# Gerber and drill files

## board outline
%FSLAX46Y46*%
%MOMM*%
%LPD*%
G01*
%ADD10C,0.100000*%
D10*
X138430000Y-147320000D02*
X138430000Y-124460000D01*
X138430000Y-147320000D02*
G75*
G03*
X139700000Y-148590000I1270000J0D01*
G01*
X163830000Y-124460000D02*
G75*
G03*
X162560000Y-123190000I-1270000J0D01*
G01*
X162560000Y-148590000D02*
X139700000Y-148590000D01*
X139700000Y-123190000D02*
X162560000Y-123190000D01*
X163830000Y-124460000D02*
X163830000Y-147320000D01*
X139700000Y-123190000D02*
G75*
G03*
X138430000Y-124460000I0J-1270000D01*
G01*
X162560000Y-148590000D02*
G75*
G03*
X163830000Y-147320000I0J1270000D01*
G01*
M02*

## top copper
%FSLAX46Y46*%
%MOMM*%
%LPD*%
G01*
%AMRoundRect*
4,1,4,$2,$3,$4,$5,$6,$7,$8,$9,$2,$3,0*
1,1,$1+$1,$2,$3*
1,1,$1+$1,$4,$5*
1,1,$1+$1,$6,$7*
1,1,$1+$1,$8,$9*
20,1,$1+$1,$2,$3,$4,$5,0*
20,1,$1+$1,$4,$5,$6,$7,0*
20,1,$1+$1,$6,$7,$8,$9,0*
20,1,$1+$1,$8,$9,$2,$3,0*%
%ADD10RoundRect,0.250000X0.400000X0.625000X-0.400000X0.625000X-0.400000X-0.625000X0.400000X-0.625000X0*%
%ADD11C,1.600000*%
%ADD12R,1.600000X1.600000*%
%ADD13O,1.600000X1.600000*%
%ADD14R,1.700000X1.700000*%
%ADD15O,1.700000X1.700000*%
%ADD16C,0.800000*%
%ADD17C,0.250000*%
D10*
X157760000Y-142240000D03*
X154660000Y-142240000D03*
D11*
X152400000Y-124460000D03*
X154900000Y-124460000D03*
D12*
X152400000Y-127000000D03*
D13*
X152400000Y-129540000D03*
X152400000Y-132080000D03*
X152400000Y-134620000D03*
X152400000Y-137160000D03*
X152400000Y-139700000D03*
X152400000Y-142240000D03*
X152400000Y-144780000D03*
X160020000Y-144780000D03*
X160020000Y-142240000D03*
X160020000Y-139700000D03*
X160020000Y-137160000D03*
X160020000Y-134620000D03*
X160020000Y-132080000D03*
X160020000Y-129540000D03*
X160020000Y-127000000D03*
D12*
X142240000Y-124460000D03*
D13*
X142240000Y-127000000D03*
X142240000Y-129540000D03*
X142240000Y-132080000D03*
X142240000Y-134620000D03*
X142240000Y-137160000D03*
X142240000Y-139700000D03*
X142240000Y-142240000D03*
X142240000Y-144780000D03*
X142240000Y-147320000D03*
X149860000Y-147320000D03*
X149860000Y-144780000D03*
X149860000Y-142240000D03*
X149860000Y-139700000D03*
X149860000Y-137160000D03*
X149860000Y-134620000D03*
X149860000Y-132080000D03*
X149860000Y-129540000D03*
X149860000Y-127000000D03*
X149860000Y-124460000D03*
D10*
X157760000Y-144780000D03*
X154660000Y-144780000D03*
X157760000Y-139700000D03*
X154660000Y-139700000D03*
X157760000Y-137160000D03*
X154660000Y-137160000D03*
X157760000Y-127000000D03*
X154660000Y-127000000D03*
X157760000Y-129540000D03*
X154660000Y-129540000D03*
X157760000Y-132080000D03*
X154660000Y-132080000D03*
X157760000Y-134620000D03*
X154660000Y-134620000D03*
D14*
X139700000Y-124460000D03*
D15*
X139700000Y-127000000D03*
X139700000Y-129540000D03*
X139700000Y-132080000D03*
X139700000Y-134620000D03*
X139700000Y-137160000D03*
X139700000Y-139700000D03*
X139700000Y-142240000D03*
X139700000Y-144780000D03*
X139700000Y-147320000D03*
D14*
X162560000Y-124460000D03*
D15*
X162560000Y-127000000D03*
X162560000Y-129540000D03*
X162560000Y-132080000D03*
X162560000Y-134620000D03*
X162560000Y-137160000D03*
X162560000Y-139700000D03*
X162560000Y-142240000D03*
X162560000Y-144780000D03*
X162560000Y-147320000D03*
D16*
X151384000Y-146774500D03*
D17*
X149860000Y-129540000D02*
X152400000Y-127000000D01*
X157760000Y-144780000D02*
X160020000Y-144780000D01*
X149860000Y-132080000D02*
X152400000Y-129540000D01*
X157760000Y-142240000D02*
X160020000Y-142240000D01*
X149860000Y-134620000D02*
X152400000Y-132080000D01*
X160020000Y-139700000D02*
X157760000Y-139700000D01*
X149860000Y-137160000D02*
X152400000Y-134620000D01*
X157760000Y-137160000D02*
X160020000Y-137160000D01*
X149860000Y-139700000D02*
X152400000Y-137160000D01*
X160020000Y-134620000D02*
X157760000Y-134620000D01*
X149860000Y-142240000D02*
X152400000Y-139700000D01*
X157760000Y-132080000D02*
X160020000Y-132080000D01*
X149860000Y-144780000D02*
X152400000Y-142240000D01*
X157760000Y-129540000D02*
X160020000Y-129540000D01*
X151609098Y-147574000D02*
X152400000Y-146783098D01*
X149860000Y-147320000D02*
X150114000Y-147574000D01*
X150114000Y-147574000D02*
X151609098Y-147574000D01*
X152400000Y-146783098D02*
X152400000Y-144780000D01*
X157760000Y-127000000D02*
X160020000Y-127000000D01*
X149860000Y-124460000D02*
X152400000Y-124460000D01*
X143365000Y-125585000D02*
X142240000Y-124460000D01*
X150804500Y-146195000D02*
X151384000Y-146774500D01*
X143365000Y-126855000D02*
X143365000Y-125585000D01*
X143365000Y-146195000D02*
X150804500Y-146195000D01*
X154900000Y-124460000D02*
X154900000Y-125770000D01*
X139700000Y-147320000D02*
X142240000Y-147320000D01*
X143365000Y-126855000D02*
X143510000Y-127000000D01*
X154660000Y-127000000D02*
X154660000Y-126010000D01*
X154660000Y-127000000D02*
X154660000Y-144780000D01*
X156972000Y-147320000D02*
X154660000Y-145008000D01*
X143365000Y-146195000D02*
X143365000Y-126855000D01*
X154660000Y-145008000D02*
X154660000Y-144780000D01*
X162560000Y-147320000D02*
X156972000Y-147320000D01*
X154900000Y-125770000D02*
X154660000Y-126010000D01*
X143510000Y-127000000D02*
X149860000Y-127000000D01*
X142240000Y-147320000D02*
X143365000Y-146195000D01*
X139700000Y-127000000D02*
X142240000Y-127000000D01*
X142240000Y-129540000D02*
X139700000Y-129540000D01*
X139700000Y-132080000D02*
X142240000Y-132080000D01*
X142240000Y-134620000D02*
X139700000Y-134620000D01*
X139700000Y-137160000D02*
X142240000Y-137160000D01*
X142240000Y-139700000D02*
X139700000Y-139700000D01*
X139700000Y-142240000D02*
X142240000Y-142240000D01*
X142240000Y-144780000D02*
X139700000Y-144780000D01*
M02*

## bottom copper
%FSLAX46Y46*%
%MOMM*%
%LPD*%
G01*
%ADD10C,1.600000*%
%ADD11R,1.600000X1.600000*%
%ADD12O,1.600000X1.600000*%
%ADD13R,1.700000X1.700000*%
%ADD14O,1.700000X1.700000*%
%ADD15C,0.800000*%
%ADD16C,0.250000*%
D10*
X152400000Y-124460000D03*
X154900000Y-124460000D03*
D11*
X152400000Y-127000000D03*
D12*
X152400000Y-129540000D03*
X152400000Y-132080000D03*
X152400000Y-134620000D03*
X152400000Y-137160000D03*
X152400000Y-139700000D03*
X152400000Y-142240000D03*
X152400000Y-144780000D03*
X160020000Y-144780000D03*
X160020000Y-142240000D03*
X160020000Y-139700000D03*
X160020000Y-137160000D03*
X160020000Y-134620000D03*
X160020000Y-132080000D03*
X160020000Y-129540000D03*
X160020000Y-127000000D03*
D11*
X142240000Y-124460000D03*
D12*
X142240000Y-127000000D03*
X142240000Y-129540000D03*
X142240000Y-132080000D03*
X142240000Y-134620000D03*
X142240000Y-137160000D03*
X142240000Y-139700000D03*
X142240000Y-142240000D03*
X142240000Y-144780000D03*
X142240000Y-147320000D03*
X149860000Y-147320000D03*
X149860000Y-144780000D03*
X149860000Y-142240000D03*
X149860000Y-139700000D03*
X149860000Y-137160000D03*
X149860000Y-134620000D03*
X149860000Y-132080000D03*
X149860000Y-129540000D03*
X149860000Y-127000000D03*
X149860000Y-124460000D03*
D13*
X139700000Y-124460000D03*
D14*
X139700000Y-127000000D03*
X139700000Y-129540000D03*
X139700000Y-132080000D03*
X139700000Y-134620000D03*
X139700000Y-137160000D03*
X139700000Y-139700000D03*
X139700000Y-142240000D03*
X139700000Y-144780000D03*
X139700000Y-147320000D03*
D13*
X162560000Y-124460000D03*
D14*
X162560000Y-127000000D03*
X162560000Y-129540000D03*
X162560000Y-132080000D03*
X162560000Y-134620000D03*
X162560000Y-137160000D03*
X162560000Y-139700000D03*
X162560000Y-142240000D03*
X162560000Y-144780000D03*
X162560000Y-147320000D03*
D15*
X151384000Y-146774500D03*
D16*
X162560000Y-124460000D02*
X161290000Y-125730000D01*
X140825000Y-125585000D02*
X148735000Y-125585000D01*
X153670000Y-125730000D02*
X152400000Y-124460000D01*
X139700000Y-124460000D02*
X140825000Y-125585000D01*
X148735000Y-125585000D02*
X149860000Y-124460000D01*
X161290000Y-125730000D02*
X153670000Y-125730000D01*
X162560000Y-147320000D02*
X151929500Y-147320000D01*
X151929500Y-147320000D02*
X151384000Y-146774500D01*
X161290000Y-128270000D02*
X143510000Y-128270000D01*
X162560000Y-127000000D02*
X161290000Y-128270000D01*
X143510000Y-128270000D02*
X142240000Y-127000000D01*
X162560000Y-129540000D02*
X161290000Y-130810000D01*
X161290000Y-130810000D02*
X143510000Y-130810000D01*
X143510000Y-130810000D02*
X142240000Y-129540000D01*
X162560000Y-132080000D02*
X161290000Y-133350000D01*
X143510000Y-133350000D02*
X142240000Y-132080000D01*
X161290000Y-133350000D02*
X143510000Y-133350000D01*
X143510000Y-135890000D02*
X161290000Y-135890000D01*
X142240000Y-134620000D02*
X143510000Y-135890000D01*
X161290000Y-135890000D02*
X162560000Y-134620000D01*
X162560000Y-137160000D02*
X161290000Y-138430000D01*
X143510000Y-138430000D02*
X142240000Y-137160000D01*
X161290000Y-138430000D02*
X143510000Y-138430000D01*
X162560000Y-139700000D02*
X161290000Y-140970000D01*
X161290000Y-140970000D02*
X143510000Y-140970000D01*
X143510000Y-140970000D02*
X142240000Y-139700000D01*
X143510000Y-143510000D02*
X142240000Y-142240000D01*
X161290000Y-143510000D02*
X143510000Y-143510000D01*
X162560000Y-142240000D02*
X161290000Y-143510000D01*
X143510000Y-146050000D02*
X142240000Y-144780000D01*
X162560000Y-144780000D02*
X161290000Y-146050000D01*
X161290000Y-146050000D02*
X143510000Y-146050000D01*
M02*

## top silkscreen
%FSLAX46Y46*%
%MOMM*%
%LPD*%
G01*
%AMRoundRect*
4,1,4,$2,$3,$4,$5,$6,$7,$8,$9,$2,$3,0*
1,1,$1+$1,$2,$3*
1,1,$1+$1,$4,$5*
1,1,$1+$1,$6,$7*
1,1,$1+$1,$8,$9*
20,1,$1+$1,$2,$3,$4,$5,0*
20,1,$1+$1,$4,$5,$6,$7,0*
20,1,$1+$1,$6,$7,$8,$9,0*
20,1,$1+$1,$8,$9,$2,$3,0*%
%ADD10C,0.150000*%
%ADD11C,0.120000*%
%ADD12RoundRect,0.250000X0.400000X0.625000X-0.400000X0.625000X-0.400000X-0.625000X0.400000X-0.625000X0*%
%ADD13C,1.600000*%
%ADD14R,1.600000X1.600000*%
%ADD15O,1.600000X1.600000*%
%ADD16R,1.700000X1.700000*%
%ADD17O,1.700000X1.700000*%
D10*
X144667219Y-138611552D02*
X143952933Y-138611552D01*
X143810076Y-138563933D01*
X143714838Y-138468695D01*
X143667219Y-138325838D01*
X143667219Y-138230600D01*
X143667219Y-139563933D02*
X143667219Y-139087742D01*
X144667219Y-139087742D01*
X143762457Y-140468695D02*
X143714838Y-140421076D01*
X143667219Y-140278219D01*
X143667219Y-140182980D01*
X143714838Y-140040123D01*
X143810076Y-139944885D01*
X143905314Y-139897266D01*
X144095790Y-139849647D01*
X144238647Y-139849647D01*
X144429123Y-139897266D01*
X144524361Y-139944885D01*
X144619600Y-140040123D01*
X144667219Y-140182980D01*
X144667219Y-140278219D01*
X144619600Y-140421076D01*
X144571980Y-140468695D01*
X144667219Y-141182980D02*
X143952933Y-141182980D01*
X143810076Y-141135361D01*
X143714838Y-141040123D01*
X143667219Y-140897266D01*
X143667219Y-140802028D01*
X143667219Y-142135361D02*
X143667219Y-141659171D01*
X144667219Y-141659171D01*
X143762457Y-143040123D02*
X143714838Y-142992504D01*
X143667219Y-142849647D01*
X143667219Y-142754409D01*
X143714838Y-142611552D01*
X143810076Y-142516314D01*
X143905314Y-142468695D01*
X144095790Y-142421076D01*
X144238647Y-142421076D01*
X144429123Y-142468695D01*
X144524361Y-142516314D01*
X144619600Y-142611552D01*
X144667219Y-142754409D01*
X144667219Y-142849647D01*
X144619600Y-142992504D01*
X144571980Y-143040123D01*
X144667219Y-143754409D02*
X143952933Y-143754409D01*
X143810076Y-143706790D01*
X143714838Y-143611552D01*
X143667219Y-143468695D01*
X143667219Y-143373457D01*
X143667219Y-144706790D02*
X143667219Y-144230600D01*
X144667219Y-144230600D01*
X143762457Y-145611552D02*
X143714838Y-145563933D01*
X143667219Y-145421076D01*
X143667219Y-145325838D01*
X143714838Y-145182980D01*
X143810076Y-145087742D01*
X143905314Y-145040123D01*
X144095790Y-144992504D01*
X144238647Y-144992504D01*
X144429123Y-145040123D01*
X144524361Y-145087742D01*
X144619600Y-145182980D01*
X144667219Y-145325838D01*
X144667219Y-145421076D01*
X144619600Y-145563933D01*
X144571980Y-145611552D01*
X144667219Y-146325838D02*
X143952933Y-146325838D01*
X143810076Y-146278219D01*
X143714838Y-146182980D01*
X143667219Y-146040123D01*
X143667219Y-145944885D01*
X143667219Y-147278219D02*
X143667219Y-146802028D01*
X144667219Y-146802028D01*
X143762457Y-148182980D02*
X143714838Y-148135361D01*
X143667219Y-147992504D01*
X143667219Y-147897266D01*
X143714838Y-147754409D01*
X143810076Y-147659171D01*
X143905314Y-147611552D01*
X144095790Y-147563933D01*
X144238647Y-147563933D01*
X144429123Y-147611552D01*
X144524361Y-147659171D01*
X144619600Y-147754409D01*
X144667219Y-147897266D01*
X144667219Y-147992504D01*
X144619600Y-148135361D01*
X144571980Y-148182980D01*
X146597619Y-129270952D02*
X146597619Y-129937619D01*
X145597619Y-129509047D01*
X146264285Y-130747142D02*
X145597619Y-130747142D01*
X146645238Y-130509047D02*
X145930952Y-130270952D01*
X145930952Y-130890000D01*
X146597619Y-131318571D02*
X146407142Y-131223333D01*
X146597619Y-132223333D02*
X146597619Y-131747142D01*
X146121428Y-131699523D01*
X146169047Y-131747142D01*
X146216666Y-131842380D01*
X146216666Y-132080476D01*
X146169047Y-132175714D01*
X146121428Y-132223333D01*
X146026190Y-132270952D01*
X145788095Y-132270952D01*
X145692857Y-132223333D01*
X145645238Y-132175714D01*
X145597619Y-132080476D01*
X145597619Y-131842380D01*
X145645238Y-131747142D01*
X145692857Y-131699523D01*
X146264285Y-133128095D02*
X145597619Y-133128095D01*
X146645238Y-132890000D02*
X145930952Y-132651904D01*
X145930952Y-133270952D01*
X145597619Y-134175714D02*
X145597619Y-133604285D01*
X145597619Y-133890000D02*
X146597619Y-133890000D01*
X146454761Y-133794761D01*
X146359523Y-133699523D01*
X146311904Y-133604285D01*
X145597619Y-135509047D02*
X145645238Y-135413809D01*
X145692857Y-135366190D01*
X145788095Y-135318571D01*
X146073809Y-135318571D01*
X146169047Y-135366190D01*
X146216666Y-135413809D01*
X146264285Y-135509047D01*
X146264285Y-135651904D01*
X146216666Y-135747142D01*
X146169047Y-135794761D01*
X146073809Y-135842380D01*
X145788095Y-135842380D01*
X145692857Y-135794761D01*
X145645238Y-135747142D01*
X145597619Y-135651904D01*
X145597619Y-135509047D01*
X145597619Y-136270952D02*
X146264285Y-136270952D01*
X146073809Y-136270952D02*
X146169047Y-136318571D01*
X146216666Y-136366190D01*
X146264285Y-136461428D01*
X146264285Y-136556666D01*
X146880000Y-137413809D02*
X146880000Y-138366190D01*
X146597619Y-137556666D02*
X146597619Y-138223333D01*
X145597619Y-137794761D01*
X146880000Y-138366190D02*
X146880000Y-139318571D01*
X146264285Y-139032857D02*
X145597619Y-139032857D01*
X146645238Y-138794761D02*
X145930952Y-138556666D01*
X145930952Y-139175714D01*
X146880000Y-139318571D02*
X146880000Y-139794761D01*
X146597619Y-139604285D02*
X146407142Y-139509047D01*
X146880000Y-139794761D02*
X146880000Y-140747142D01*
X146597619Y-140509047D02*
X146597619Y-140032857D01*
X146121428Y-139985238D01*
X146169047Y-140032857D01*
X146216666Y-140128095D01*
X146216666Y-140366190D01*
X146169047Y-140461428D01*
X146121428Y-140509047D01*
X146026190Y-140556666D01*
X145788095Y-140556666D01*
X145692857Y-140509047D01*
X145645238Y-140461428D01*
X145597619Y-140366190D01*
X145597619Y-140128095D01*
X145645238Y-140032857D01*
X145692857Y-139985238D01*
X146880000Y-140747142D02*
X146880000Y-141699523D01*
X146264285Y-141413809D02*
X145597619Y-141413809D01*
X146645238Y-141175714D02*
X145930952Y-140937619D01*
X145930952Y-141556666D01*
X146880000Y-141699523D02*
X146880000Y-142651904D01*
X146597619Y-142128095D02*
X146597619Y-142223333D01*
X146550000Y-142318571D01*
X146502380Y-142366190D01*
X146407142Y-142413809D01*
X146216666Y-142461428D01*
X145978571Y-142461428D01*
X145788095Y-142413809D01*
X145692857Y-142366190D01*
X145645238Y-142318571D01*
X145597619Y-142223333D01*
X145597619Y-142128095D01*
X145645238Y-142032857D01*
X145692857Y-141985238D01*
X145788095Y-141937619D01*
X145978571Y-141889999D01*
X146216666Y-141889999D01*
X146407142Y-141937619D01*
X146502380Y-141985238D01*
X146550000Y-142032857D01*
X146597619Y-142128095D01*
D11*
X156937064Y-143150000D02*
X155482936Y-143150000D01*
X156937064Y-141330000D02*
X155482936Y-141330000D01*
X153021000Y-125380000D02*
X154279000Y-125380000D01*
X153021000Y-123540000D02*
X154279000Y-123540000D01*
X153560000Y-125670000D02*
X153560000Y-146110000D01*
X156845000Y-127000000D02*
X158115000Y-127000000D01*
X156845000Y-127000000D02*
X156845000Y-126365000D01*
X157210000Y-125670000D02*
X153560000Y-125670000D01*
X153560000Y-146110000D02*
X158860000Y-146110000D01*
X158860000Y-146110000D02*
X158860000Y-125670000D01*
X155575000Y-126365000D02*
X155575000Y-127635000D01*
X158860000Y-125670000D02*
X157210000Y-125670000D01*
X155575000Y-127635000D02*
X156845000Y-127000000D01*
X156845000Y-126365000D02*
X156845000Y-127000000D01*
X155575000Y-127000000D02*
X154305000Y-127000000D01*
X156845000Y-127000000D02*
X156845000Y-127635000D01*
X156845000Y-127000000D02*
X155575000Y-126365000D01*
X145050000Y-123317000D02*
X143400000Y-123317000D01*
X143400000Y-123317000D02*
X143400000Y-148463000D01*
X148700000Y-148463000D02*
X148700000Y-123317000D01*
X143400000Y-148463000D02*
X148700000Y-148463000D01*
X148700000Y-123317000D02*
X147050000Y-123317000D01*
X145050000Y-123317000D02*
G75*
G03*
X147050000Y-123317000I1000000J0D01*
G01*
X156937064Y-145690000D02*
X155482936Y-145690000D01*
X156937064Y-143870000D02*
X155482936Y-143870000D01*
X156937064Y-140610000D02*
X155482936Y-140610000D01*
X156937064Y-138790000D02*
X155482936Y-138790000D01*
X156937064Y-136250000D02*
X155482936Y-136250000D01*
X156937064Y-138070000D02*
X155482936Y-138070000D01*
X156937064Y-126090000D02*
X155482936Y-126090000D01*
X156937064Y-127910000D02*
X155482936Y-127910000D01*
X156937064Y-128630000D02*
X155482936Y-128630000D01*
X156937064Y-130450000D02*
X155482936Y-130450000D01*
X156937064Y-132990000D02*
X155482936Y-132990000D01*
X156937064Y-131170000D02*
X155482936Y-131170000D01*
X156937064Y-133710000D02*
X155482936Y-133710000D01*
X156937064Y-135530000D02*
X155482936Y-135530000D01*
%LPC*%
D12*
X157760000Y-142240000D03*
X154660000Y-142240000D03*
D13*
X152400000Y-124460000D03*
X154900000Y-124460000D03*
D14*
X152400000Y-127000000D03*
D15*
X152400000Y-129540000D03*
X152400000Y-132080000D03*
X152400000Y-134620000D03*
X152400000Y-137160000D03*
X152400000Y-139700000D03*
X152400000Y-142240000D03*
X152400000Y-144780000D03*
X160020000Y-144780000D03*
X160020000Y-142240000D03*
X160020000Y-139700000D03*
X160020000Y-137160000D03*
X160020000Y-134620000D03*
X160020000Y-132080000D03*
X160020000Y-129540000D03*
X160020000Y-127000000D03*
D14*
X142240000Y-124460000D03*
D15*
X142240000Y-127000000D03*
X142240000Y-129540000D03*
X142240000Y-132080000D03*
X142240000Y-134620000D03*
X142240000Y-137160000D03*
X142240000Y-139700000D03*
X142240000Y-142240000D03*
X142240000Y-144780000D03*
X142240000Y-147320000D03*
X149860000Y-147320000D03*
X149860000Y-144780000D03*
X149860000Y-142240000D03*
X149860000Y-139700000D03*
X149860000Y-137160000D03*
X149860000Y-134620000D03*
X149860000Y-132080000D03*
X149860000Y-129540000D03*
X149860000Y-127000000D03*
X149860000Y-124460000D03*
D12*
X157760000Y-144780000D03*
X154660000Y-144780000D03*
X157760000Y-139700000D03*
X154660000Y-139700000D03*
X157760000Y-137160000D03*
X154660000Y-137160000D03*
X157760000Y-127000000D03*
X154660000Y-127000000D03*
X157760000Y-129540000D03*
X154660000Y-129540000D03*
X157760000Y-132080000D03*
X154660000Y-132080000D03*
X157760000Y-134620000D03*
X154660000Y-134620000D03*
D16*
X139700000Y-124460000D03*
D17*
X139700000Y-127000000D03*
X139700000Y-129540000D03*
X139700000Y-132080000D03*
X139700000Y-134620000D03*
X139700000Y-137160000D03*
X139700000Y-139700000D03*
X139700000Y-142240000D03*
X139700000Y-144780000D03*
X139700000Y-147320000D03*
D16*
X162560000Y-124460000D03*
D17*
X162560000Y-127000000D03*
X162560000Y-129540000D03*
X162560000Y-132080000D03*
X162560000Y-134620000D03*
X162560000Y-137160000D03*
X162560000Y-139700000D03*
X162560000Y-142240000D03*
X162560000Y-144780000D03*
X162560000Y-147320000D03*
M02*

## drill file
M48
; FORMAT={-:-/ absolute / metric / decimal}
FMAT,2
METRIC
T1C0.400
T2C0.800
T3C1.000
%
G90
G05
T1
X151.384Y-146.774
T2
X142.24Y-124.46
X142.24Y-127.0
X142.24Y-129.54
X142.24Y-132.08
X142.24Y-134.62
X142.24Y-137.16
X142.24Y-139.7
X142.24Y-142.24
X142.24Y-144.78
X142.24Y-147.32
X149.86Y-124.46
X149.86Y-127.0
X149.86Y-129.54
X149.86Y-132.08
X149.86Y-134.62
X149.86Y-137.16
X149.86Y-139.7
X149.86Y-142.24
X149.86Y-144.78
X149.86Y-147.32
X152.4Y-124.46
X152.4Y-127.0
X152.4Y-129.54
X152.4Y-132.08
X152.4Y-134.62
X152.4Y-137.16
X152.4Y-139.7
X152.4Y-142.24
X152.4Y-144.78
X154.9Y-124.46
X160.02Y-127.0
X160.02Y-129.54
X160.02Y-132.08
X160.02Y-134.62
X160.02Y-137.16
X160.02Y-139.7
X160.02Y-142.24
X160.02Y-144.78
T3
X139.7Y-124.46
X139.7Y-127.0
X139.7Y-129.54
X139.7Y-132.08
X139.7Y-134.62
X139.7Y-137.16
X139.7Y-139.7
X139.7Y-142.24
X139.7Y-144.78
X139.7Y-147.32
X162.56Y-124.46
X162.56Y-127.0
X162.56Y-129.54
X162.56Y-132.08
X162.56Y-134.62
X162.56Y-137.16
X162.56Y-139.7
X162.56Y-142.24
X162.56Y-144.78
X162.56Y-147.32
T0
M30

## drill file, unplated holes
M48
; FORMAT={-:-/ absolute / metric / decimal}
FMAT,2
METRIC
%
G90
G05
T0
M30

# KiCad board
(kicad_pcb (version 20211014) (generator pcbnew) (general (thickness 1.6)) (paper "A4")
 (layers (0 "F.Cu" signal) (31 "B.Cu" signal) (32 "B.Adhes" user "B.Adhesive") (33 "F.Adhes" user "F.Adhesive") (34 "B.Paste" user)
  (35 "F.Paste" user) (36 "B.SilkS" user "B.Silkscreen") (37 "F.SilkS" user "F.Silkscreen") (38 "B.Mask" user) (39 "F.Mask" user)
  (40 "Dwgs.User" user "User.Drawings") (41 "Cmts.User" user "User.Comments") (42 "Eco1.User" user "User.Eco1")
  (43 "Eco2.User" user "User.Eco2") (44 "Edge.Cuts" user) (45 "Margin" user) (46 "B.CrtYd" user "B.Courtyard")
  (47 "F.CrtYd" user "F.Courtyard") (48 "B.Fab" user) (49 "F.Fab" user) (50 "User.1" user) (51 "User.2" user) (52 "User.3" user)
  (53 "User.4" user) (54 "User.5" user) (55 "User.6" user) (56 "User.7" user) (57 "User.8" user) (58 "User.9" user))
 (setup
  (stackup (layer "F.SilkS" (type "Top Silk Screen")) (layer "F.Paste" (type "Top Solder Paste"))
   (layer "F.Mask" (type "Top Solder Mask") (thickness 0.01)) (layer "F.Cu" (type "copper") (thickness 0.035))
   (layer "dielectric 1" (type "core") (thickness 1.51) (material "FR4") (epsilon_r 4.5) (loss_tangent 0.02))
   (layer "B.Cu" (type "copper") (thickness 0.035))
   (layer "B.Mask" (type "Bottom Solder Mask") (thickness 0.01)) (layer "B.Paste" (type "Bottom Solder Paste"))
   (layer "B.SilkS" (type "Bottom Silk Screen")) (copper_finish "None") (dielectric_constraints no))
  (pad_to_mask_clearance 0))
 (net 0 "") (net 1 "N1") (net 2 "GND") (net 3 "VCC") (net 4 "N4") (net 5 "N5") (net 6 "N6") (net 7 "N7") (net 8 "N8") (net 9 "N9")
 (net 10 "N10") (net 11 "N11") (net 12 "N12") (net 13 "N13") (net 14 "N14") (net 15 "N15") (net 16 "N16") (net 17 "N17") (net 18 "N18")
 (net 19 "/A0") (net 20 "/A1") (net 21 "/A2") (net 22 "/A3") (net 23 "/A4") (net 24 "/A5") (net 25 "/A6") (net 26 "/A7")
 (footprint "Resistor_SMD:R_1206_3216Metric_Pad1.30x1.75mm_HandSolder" (layer "F.Cu") (at 156.21 142.24 180)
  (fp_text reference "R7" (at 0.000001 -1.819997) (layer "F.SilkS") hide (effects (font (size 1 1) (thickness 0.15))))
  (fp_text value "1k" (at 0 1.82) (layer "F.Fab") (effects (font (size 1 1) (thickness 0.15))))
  (fp_line (start -0.727064 -0.91) (end 0.727064 -0.91) (layer "F.SilkS") (width 0.12))
  (fp_line (start -0.727064 0.91) (end 0.727064 0.91) (layer "F.SilkS") (width 0.12))
  (pad "1" smd roundrect locked (at -1.55 0 180) (size 1.3 1.75) (layers "F.Cu" "F.Paste" "F.Mask") (roundrect_rratio 0.1923076923)
   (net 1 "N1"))
  (pad "2" smd roundrect locked (at 1.55 0 180) (size 1.3 1.75) (layers "F.Cu" "F.Paste" "F.Mask") (roundrect_rratio 0.1923076923)
   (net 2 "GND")))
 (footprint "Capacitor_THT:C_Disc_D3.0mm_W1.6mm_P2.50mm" (layer "F.Cu") (at 152.4 124.46)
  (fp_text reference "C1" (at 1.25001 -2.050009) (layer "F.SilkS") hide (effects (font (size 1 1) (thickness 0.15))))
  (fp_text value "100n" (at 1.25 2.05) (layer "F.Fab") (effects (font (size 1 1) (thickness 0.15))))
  (fp_line (start 0.621 0.92) (end 1.879 0.92) (layer "F.SilkS") (width 0.12))
  (fp_line (start 0.621 -0.92) (end 1.879 -0.92) (layer "F.SilkS") (width 0.12))
  (pad "1" thru_hole circle locked (at 0 0) (size 1.6 1.6) (drill 0.8) (layers *.Cu *.Mask) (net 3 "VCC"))
  (pad "2" thru_hole circle locked (at 2.5 0) (size 1.6 1.6) (drill 0.8) (layers *.Cu *.Mask) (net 2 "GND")))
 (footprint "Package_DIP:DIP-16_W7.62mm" (layer "F.Cu") (at 152.4 127)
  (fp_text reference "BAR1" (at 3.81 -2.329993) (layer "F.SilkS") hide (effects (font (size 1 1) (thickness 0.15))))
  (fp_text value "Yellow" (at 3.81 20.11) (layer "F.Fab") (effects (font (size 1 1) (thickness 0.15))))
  (fp_line (start 1.16 -1.33) (end 1.16 19.11) (layer "F.SilkS") (width 0.12))
  (fp_line (start 4.445 0) (end 5.715 0) (layer "F.SilkS") (width 0.12))
  (fp_line (start 4.445 0) (end 4.445 -0.635) (layer "F.SilkS") (width 0.12))
  (fp_line (start 4.81 -1.33) (end 1.16 -1.33) (layer "F.SilkS") (width 0.12))
  (fp_line (start 1.16 19.11) (end 6.46 19.11) (layer "F.SilkS") (width 0.12))
  (fp_line (start 6.46 19.11) (end 6.46 -1.33) (layer "F.SilkS") (width 0.12))
  (fp_line (start 3.175 -0.635) (end 3.175 0.635) (layer "F.SilkS") (width 0.12))
  (fp_line (start 6.46 -1.33) (end 4.81 -1.33) (layer "F.SilkS") (width 0.12))
  (fp_line (start 3.175 0.635) (end 4.445 0) (layer "F.SilkS") (width 0.12))
  (fp_line (start 4.445 -0.635) (end 4.445 0) (layer "F.SilkS") (width 0.12))
  (fp_line (start 3.175 0) (end 1.905 0) (layer "F.SilkS") (width 0.12))
  (fp_line (start 4.445 0) (end 4.445 0.635) (layer "F.SilkS") (width 0.12))
  (fp_line (start 4.445 0) (end 3.175 -0.635) (layer "F.SilkS") (width 0.12))
  (pad "1" thru_hole rect (at 0 0) (size 1.6 1.6) (drill 0.8) (layers *.Cu *.Mask) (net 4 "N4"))
  (pad "2" thru_hole oval (at 0 2.54) (size 1.6 1.6) (drill 0.8) (layers *.Cu *.Mask) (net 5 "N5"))
  (pad "3" thru_hole oval (at 0 5.08) (size 1.6 1.6) (drill 0.8) (layers *.Cu *.Mask) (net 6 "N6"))
  (pad "4" thru_hole oval (at 0 7.62) (size 1.6 1.6) (drill 0.8) (layers *.Cu *.Mask) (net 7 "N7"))
  (pad "5" thru_hole oval (at 0 10.16) (size 1.6 1.6) (drill 0.8) (layers *.Cu *.Mask) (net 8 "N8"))
  (pad "6" thru_hole oval (at 0 12.7) (size 1.6 1.6) (drill 0.8) (layers *.Cu *.Mask) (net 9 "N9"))
  (pad "7" thru_hole oval (at 0 15.24) (size 1.6 1.6) (drill 0.8) (layers *.Cu *.Mask) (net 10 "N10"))
  (pad "8" thru_hole oval (at 0 17.78) (size 1.6 1.6) (drill 0.8) (layers *.Cu *.Mask) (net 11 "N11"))
  (pad "9" thru_hole oval (at 7.62 17.78) (size 1.6 1.6) (drill 0.8) (layers *.Cu *.Mask) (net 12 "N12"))
  (pad "10" thru_hole oval (at 7.62 15.24) (size 1.6 1.6) (drill 0.8) (layers *.Cu *.Mask) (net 1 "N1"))
  (pad "11" thru_hole oval (at 7.62 12.7) (size 1.6 1.6) (drill 0.8) (layers *.Cu *.Mask) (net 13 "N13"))
  (pad "12" thru_hole oval (at 7.62 10.16) (size 1.6 1.6) (drill 0.8) (layers *.Cu *.Mask) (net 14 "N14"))
  (pad "13" thru_hole oval (at 7.62 7.62) (size 1.6 1.6) (drill 0.8) (layers *.Cu *.Mask) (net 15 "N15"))
  (pad "14" thru_hole oval (at 7.62 5.08) (size 1.6 1.6) (drill 0.8) (layers *.Cu *.Mask) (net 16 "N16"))
  (pad "15" thru_hole oval (at 7.62 2.54) (size 1.6 1.6) (drill 0.8) (layers *.Cu *.Mask) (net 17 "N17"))
  (pad "16" thru_hole oval (at 7.62 0) (size 1.6 1.6) (drill 0.8) (layers *.Cu *.Mask) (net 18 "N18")))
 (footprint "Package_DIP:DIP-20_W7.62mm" (layer "F.Cu") (at 142.24 124.46)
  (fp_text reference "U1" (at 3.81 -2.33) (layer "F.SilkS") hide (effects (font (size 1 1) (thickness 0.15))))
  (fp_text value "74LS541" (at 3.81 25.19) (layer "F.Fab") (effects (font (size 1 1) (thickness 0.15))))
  (fp_line (start 2.81 -1.143) (end 1.16 -1.143) (layer "F.SilkS") (width 0.12))
  (fp_line (start 1.16 -1.143) (end 1.16 24.003) (layer "F.SilkS") (width 0.12))
  (fp_line (start 6.46 24.003) (end 6.46 -1.143) (layer "F.SilkS") (width 0.12))
  (fp_line (start 1.16 24.003) (end 6.46 24.003) (layer "F.SilkS") (width 0.12))
  (fp_line (start 6.46 -1.143) (end 4.81 -1.143) (layer "F.SilkS") (width 0.12))
  (fp_arc (start 4.81 -1.143) (mid 3.81 -0.143) (end 2.81 -1.143) (layer "F.SilkS") (width 0.12))
  (pad "1" thru_hole rect (at 0 0) (size 1.6 1.6) (drill 0.8) (layers *.Cu *.Mask) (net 2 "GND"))
  (pad "2" thru_hole oval (at 0 2.54) (size 1.6 1.6) (drill 0.8) (layers *.Cu *.Mask) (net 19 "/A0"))
  (pad "3" thru_hole oval (at 0 5.08) (size 1.6 1.6) (drill 0.8) (layers *.Cu *.Mask) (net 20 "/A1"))
  (pad "4" thru_hole oval (at 0 7.62) (size 1.6 1.6) (drill 0.8) (layers *.Cu *.Mask) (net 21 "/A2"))
  (pad "5" thru_hole oval (at 0 10.16) (size 1.6 1.6) (drill 0.8) (layers *.Cu *.Mask) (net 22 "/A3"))
  (pad "6" thru_hole oval (at 0 12.7) (size 1.6 1.6) (drill 0.8) (layers *.Cu *.Mask) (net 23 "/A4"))
  (pad "7" thru_hole oval (at 0 15.24) (size 1.6 1.6) (drill 0.8) (layers *.Cu *.Mask) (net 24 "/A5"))
  (pad "8" thru_hole oval (at 0 17.78) (size 1.6 1.6) (drill 0.8) (layers *.Cu *.Mask) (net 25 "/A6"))
  (pad "9" thru_hole oval (at 0 20.32) (size 1.6 1.6) (drill 0.8) (layers *.Cu *.Mask) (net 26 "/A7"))
  (pad "10" thru_hole oval (at 0 22.86) (size 1.6 1.6) (drill 0.8) (layers *.Cu *.Mask) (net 2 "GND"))
  (pad "11" thru_hole oval (at 7.62 22.86) (size 1.6 1.6) (drill 0.8) (layers *.Cu *.Mask) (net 11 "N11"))
  (pad "12" thru_hole oval (at 7.62 20.32) (size 1.6 1.6) (drill 0.8) (layers *.Cu *.Mask) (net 10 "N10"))
  (pad "13" thru_hole oval (at 7.62 17.78) (size 1.6 1.6) (drill 0.8) (layers *.Cu *.Mask) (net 9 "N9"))
  (pad "14" thru_hole oval (at 7.62 15.24) (size 1.6 1.6) (drill 0.8) (layers *.Cu *.Mask) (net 8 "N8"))
  (pad "15" thru_hole oval (at 7.62 12.7) (size 1.6 1.6) (drill 0.8) (layers *.Cu *.Mask) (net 7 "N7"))
  (pad "16" thru_hole oval (at 7.62 10.16) (size 1.6 1.6) (drill 0.8) (layers *.Cu *.Mask) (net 6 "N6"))
  (pad "17" thru_hole oval (at 7.62 7.62) (size 1.6 1.6) (drill 0.8) (layers *.Cu *.Mask) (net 5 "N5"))
  (pad "18" thru_hole oval (at 7.62 5.08) (size 1.6 1.6) (drill 0.8) (layers *.Cu *.Mask) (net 4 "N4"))
  (pad "19" thru_hole oval (at 7.62 2.54) (size 1.6 1.6) (drill 0.8) (layers *.Cu *.Mask) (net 2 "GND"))
  (pad "20" thru_hole oval (at 7.62 0) (size 1.6 1.6) (drill 0.8) (layers *.Cu *.Mask) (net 3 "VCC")))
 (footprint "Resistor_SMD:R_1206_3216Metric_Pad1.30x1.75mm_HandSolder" (layer "F.Cu") (at 156.21 144.78 180)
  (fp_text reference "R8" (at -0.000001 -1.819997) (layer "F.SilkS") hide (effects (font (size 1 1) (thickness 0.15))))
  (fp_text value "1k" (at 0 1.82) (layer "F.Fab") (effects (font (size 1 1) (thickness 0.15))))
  (fp_line (start -0.727064 -0.91) (end 0.727064 -0.91) (layer "F.SilkS") (width 0.12))
  (fp_line (start -0.727064 0.91) (end 0.727064 0.91) (layer "F.SilkS") (width 0.12))
  (pad "1" smd roundrect locked (at -1.55 0 180) (size 1.3 1.75) (layers "F.Cu" "F.Paste" "F.Mask") (roundrect_rratio 0.1923076923)
   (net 12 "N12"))
  (pad "2" smd roundrect locked (at 1.55 0 180) (size 1.3 1.75) (layers "F.Cu" "F.Paste" "F.Mask") (roundrect_rratio 0.1923076923)
   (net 2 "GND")))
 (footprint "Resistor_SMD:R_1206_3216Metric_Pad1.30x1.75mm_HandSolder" (layer "F.Cu") (at 156.21 139.7 180)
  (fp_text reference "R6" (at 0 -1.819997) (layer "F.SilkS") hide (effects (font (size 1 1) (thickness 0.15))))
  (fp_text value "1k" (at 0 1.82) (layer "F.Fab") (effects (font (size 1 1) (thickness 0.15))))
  (fp_line (start -0.727064 -0.91) (end 0.727064 -0.91) (layer "F.SilkS") (width 0.12))
  (fp_line (start -0.727064 0.91) (end 0.727064 0.91) (layer "F.SilkS") (width 0.12))
  (pad "1" smd roundrect locked (at -1.55 0 180) (size 1.3 1.75) (layers "F.Cu" "F.Paste" "F.Mask") (roundrect_rratio 0.1923076923)
   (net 13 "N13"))
  (pad "2" smd roundrect locked (at 1.55 0 180) (size 1.3 1.75) (layers "F.Cu" "F.Paste" "F.Mask") (roundrect_rratio 0.1923076923)
   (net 2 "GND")))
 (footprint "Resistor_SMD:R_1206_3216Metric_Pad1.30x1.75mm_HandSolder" (layer "F.Cu") (at 156.21 137.16 180)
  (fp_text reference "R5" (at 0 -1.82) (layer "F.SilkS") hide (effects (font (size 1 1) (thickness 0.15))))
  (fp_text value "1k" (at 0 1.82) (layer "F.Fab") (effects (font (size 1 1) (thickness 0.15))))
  (fp_line (start -0.727064 0.91) (end 0.727064 0.91) (layer "F.SilkS") (width 0.12))
  (fp_line (start -0.727064 -0.91) (end 0.727064 -0.91) (layer "F.SilkS") (width 0.12))
  (pad "1" smd roundrect locked (at -1.55 0 180) (size 1.3 1.75) (layers "F.Cu" "F.Paste" "F.Mask") (roundrect_rratio 0.1923076923)
   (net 14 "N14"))
  (pad "2" smd roundrect locked (at 1.55 0 180) (size 1.3 1.75) (layers "F.Cu" "F.Paste" "F.Mask") (roundrect_rratio 0.1923076923)
   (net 2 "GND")))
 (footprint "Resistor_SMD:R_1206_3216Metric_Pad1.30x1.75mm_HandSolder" (layer "F.Cu") (at 156.21 127 180)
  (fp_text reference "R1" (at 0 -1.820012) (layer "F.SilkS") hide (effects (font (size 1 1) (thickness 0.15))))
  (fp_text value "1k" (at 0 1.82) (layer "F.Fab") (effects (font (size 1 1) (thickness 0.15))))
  (fp_line (start -0.727064 0.91) (end 0.727064 0.91) (layer "F.SilkS") (width 0.12))
  (fp_line (start -0.727064 -0.91) (end 0.727064 -0.91) (layer "F.SilkS") (width 0.12))
  (pad "1" smd roundrect locked (at -1.55 0 180) (size 1.3 1.75) (layers "F.Cu" "F.Paste" "F.Mask") (roundrect_rratio 0.1923076923)
   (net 18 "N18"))
  (pad "2" smd roundrect locked (at 1.55 0 180) (size 1.3 1.75) (layers "F.Cu" "F.Paste" "F.Mask") (roundrect_rratio 0.1923076923)
   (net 2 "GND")))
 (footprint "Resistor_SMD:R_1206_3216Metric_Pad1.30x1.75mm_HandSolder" (layer "F.Cu") (at 156.21 129.54 180)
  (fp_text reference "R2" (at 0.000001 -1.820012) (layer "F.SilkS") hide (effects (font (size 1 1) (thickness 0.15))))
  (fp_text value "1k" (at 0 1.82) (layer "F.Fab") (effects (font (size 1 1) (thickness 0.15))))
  (fp_line (start -0.727064 0.91) (end 0.727064 0.91) (layer "F.SilkS") (width 0.12))
  (fp_line (start -0.727064 -0.91) (end 0.727064 -0.91) (layer "F.SilkS") (width 0.12))
  (pad "1" smd roundrect locked (at -1.55 0 180) (size 1.3 1.75) (layers "F.Cu" "F.Paste" "F.Mask") (roundrect_rratio 0.1923076923)
   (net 17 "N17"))
  (pad "2" smd roundrect locked (at 1.55 0 180) (size 1.3 1.75) (layers "F.Cu" "F.Paste" "F.Mask") (roundrect_rratio 0.1923076923)
   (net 2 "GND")))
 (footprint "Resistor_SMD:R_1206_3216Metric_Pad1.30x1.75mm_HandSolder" (layer "F.Cu") (at 156.21 132.08 180)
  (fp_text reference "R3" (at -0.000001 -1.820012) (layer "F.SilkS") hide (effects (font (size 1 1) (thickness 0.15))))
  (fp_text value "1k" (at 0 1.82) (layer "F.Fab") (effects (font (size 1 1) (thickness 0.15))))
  (fp_line (start -0.727064 -0.91) (end 0.727064 -0.91) (layer "F.SilkS") (width 0.12))
  (fp_line (start -0.727064 0.91) (end 0.727064 0.91) (layer "F.SilkS") (width 0.12))
  (pad "1" smd roundrect locked (at -1.55 0 180) (size 1.3 1.75) (layers "F.Cu" "F.Paste" "F.Mask") (roundrect_rratio 0.1923076923)
   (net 16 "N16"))
  (pad "2" smd roundrect locked (at 1.55 0 180) (size 1.3 1.75) (layers "F.Cu" "F.Paste" "F.Mask") (roundrect_rratio 0.1923076923)
   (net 2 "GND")))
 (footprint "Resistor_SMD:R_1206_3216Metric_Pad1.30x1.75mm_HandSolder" (layer "F.Cu") (at 156.21 134.62 180)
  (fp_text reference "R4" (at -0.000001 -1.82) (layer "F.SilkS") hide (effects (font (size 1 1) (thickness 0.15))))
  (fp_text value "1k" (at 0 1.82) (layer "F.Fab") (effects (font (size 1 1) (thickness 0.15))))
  (fp_line (start -0.727064 0.91) (end 0.727064 0.91) (layer "F.SilkS") (width 0.12))
  (fp_line (start -0.727064 -0.91) (end 0.727064 -0.91) (layer "F.SilkS") (width 0.12))
  (pad "1" smd roundrect locked (at -1.55 0 180) (size 1.3 1.75) (layers "F.Cu" "F.Paste" "F.Mask") (roundrect_rratio 0.1923076923)
   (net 15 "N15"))
  (pad "2" smd roundrect locked (at 1.55 0 180) (size 1.3 1.75) (layers "F.Cu" "F.Paste" "F.Mask") (roundrect_rratio 0.1923076923)
   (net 2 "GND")))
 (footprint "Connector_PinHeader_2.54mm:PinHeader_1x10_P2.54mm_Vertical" (layer "B.Cu") (at 139.7 124.46 180)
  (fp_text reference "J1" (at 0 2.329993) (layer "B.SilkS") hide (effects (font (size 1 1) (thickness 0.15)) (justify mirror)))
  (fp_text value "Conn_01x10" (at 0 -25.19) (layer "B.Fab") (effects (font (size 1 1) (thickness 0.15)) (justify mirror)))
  (pad "1" thru_hole rect (at 0 0 180) (size 1.7 1.7) (drill 1) (layers *.Cu *.Mask) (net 3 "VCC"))
  (pad "2" thru_hole oval (at 0 -2.54 180) (size 1.7 1.7) (drill 1) (layers *.Cu *.Mask) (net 19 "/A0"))
  (pad "3" thru_hole oval (at 0 -5.08 180) (size 1.7 1.7) (drill 1) (layers *.Cu *.Mask) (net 20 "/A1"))
  (pad "4" thru_hole oval (at 0 -7.62 180) (size 1.7 1.7) (drill 1) (layers *.Cu *.Mask) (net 21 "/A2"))
  (pad "5" thru_hole oval (at 0 -10.16 180) (size 1.7 1.7) (drill 1) (layers *.Cu *.Mask) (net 22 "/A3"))
  (pad "6" thru_hole oval (at 0 -12.7 180) (size 1.7 1.7) (drill 1) (layers *.Cu *.Mask) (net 23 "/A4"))
  (pad "7" thru_hole oval (at 0 -15.24 180) (size 1.7 1.7) (drill 1) (layers *.Cu *.Mask) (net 24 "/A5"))
  (pad "8" thru_hole oval (at 0 -17.78 180) (size 1.7 1.7) (drill 1) (layers *.Cu *.Mask) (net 25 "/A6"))
  (pad "9" thru_hole oval (at 0 -20.32 180) (size 1.7 1.7) (drill 1) (layers *.Cu *.Mask) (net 26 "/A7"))
  (pad "10" thru_hole oval (at 0 -22.86 180) (size 1.7 1.7) (drill 1) (layers *.Cu *.Mask) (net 2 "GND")))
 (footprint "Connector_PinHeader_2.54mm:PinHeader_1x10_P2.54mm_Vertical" (layer "B.Cu") (at 162.56 124.46 180)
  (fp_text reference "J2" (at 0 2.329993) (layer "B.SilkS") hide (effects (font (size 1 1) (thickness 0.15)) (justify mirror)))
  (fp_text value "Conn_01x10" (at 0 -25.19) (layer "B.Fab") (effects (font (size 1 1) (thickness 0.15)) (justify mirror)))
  (pad "1" thru_hole rect (at 0 0 180) (size 1.7 1.7) (drill 1) (layers *.Cu *.Mask) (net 3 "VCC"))
  (pad "2" thru_hole oval (at 0 -2.54 180) (size 1.7 1.7) (drill 1) (layers *.Cu *.Mask) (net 19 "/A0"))
  (pad "3" thru_hole oval (at 0 -5.08 180) (size 1.7 1.7) (drill 1) (layers *.Cu *.Mask) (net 20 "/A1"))
  (pad "4" thru_hole oval (at 0 -7.62 180) (size 1.7 1.7) (drill 1) (layers *.Cu *.Mask) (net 21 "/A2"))
  (pad "5" thru_hole oval (at 0 -10.16 180) (size 1.7 1.7) (drill 1) (layers *.Cu *.Mask) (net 22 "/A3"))
  (pad "6" thru_hole oval (at 0 -12.7 180) (size 1.7 1.7) (drill 1) (layers *.Cu *.Mask) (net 23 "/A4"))
  (pad "7" thru_hole oval (at 0 -15.24 180) (size 1.7 1.7) (drill 1) (layers *.Cu *.Mask) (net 24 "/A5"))
  (pad "8" thru_hole oval (at 0 -17.78 180) (size 1.7 1.7) (drill 1) (layers *.Cu *.Mask) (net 25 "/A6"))
  (pad "9" thru_hole oval (at 0 -20.32 180) (size 1.7 1.7) (drill 1) (layers *.Cu *.Mask) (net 26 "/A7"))
  (pad "10" thru_hole oval (at 0 -22.86 180) (size 1.7 1.7) (drill 1) (layers *.Cu *.Mask) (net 2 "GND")))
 (gr_line (start 138.43 147.32) (end 138.43 124.46) (layer "Edge.Cuts") (width 0.1))
 (gr_arc (start 139.7 148.59) (mid 138.801974 148.218026) (end 138.43 147.32) (layer "Edge.Cuts") (width 0.1))
 (gr_arc (start 162.56 123.19) (mid 163.458026 123.561974) (end 163.83 124.46) (layer "Edge.Cuts") (width 0.1))
 (gr_line (start 162.56 148.59) (end 139.7 148.59) (layer "Edge.Cuts") (width 0.1))
 (gr_line (start 139.7 123.19) (end 162.56 123.19) (layer "Edge.Cuts") (width 0.1))
 (gr_line (start 163.83 124.46) (end 163.83 147.32) (layer "Edge.Cuts") (width 0.1))
 (gr_arc (start 138.43 124.46) (mid 138.801974 123.561974) (end 139.7 123.19) (layer "Edge.Cuts") (width 0.1))
 (gr_arc (start 163.83 147.32) (mid 163.458026 148.218026) (end 162.56 148.59) (layer "Edge.Cuts") (width 0.1))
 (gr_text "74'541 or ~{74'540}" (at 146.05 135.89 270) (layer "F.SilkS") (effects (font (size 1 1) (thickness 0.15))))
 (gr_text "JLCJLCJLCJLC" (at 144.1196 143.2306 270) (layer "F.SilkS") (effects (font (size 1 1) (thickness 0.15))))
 (segment (start 149.86 129.54) (end 152.4 127) (width 0.25) (layer "F.Cu") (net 4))
 (segment (start 157.76 144.78) (end 160.02 144.78) (width 0.25) (layer "F.Cu") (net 12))
 (segment (start 149.86 132.08) (end 152.4 129.54) (width 0.25) (layer "F.Cu") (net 5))
 (segment (start 157.76 142.24) (end 160.02 142.24) (width 0.25) (layer "F.Cu") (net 1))
 (segment (start 149.86 134.62) (end 152.4 132.08) (width 0.25) (layer "F.Cu") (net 6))
 (segment (start 160.02 139.7) (end 157.76 139.7) (width 0.25) (layer "F.Cu") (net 13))
 (segment (start 149.86 137.16) (end 152.4 134.62) (width 0.25) (layer "F.Cu") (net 7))
 (segment (start 157.76 137.16) (end 160.02 137.16) (width 0.25) (layer "F.Cu") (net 14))
 (segment (start 149.86 139.7) (end 152.4 137.16) (width 0.25) (layer "F.Cu") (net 8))
 (segment (start 160.02 134.62) (end 157.76 134.62) (width 0.25) (layer "F.Cu") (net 15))
 (segment (start 149.86 142.24) (end 152.4 139.7) (width 0.25) (layer "F.Cu") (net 9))
 (segment (start 157.76 132.08) (end 160.02 132.08) (width 0.25) (layer "F.Cu") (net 16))
 (segment (start 149.86 144.78) (end 152.4 142.24) (width 0.25) (layer "F.Cu") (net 10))
 (segment (start 157.76 129.54) (end 160.02 129.54) (width 0.25) (layer "F.Cu") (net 17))
 (segment (start 151.609098 147.574) (end 152.4 146.783098) (width 0.25) (layer "F.Cu") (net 11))
 (segment (start 149.86 147.32) (end 150.114 147.574) (width 0.25) (layer "F.Cu") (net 11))
 (segment (start 150.114 147.574) (end 151.609098 147.574) (width 0.25) (layer "F.Cu") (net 11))
 (segment (start 152.4 146.783098) (end 152.4 144.78) (width 0.25) (layer "F.Cu") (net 11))
 (segment (start 157.76 127) (end 160.02 127) (width 0.25) (layer "F.Cu") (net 18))
 (segment (start 149.86 124.46) (end 152.4 124.46) (width 0.25) (layer "F.Cu") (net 3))
 (segment (start 162.56 124.46) (end 161.29 125.73) (width 0.25) (layer "B.Cu") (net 3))
 (segment (start 140.825 125.585) (end 148.735 125.585) (width 0.25) (layer "B.Cu") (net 3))
 (segment (start 153.67 125.73) (end 152.4 124.46) (width 0.25) (layer "B.Cu") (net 3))
 (segment (start 139.7 124.46) (end 140.825 125.585) (width 0.25) (layer "B.Cu") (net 3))
 (segment (start 148.735 125.585) (end 149.86 124.46) (width 0.25) (layer "B.Cu") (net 3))
 (segment (start 161.29 125.73) (end 153.67 125.73) (width 0.25) (layer "B.Cu") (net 3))
 (segment (start 143.365 125.585) (end 142.24 124.46) (width 0.25) (layer "F.Cu") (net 2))
 (segment (start 150.8045 146.195) (end 151.384 146.7745) (width 0.25) (layer "F.Cu") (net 2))
 (segment (start 143.365 126.855) (end 143.365 125.585) (width 0.25) (layer "F.Cu") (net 2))
 (segment (start 143.365 146.195) (end 150.8045 146.195) (width 0.25) (layer "F.Cu") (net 2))
 (segment (start 154.9 124.46) (end 154.9 125.77) (width 0.25) (layer "F.Cu") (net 2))
 (segment (start 139.7 147.32) (end 142.24 147.32) (width 0.25) (layer "F.Cu") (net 2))
 (segment (start 143.365 126.855) (end 143.51 127) (width 0.25) (layer "F.Cu") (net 2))
 (segment (start 154.66 127) (end 154.66 126.01) (width 0.25) (layer "F.Cu") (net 2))
 (segment (start 154.66 127) (end 154.66 144.78) (width 0.25) (layer "F.Cu") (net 2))
 (segment (start 156.972 147.32) (end 154.66 145.008) (width 0.25) (layer "F.Cu") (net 2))
 (segment (start 143.365 146.195) (end 143.365 126.855) (width 0.25) (layer "F.Cu") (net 2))
 (segment (start 154.66 145.008) (end 154.66 144.78) (width 0.25) (layer "F.Cu") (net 2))
 (segment (start 162.56 147.32) (end 156.972 147.32) (width 0.25) (layer "F.Cu") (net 2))
 (segment (start 154.9 125.77) (end 154.66 126.01) (width 0.25) (layer "F.Cu") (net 2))
 (segment (start 143.51 127) (end 149.86 127) (width 0.25) (layer "F.Cu") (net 2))
 (segment (start 142.24 147.32) (end 143.365 146.195) (width 0.25) (layer "F.Cu") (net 2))
 (via (at 151.384 146.7745) (size 0.8) (drill 0.4) (layers "F.Cu" "B.Cu") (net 2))
 (segment (start 162.56 147.32) (end 151.9295 147.32) (width 0.25) (layer "B.Cu") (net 2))
 (segment (start 151.9295 147.32) (end 151.384 146.7745) (width 0.25) (layer "B.Cu") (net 2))
 (segment (start 139.7 127) (end 142.24 127) (width 0.25) (layer "F.Cu") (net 19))
 (segment (start 161.29 128.27) (end 143.51 128.27) (width 0.25) (layer "B.Cu") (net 19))
 (segment (start 162.56 127) (end 161.29 128.27) (width 0.25) (layer "B.Cu") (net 19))
 (segment (start 143.51 128.27) (end 142.24 127) (width 0.25) (layer "B.Cu") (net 19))
 (segment (start 142.24 129.54) (end 139.7 129.54) (width 0.25) (layer "F.Cu") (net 20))
 (segment (start 162.56 129.54) (end 161.29 130.81) (width 0.25) (layer "B.Cu") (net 20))
 (segment (start 161.29 130.81) (end 143.51 130.81) (width 0.25) (layer "B.Cu") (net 20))
 (segment (start 143.51 130.81) (end 142.24 129.54) (width 0.25) (layer "B.Cu") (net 20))
 (segment (start 139.7 132.08) (end 142.24 132.08) (width 0.25) (layer "F.Cu") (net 21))
 (segment (start 162.56 132.08) (end 161.29 133.35) (width 0.25) (layer "B.Cu") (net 21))
 (segment (start 143.51 133.35) (end 142.24 132.08) (width 0.25) (layer "B.Cu") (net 21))
 (segment (start 161.29 133.35) (end 143.51 133.35) (width 0.25) (layer "B.Cu") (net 21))
 (segment (start 142.24 134.62) (end 139.7 134.62) (width 0.25) (layer "F.Cu") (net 22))
 (segment (start 143.51 135.89) (end 161.29 135.89) (width 0.25) (layer "B.Cu") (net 22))
 (segment (start 142.24 134.62) (end 143.51 135.89) (width 0.25) (layer "B.Cu") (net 22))
 (segment (start 161.29 135.89) (end 162.56 134.62) (width 0.25) (layer "B.Cu") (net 22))
 (segment (start 139.7 137.16) (end 142.24 137.16) (width 0.25) (layer "F.Cu") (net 23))
 (segment (start 162.56 137.16) (end 161.29 138.43) (width 0.25) (layer "B.Cu") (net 23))
 (segment (start 143.51 138.43) (end 142.24 137.16) (width 0.25) (layer "B.Cu") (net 23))
 (segment (start 161.29 138.43) (end 143.51 138.43) (width 0.25) (layer "B.Cu") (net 23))
 (segment (start 142.24 139.7) (end 139.7 139.7) (width 0.25) (layer "F.Cu") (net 24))
 (segment (start 162.56 139.7) (end 161.29 140.97) (width 0.25) (layer "B.Cu") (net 24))
 (segment (start 161.29 140.97) (end 143.51 140.97) (width 0.25) (layer "B.Cu") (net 24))
 (segment (start 143.51 140.97) (end 142.24 139.7) (width 0.25) (layer "B.Cu") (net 24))
 (segment (start 139.7 142.24) (end 142.24 142.24) (width 0.25) (layer "F.Cu") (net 25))
 (segment (start 143.51 143.51) (end 142.24 142.24) (width 0.25) (layer "B.Cu") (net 25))
 (segment (start 161.29 143.51) (end 143.51 143.51) (width 0.25) (layer "B.Cu") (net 25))
 (segment (start 162.56 142.24) (end 161.29 143.51) (width 0.25) (layer "B.Cu") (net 25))
 (segment (start 142.24 144.78) (end 139.7 144.78) (width 0.25) (layer "F.Cu") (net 26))
 (segment (start 143.51 146.05) (end 142.24 144.78) (width 0.25) (layer "B.Cu") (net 26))
 (segment (start 162.56 144.78) (end 161.29 146.05) (width 0.25) (layer "B.Cu") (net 26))
 (segment (start 161.29 146.05) (end 143.51 146.05) (width 0.25) (layer "B.Cu") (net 26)))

